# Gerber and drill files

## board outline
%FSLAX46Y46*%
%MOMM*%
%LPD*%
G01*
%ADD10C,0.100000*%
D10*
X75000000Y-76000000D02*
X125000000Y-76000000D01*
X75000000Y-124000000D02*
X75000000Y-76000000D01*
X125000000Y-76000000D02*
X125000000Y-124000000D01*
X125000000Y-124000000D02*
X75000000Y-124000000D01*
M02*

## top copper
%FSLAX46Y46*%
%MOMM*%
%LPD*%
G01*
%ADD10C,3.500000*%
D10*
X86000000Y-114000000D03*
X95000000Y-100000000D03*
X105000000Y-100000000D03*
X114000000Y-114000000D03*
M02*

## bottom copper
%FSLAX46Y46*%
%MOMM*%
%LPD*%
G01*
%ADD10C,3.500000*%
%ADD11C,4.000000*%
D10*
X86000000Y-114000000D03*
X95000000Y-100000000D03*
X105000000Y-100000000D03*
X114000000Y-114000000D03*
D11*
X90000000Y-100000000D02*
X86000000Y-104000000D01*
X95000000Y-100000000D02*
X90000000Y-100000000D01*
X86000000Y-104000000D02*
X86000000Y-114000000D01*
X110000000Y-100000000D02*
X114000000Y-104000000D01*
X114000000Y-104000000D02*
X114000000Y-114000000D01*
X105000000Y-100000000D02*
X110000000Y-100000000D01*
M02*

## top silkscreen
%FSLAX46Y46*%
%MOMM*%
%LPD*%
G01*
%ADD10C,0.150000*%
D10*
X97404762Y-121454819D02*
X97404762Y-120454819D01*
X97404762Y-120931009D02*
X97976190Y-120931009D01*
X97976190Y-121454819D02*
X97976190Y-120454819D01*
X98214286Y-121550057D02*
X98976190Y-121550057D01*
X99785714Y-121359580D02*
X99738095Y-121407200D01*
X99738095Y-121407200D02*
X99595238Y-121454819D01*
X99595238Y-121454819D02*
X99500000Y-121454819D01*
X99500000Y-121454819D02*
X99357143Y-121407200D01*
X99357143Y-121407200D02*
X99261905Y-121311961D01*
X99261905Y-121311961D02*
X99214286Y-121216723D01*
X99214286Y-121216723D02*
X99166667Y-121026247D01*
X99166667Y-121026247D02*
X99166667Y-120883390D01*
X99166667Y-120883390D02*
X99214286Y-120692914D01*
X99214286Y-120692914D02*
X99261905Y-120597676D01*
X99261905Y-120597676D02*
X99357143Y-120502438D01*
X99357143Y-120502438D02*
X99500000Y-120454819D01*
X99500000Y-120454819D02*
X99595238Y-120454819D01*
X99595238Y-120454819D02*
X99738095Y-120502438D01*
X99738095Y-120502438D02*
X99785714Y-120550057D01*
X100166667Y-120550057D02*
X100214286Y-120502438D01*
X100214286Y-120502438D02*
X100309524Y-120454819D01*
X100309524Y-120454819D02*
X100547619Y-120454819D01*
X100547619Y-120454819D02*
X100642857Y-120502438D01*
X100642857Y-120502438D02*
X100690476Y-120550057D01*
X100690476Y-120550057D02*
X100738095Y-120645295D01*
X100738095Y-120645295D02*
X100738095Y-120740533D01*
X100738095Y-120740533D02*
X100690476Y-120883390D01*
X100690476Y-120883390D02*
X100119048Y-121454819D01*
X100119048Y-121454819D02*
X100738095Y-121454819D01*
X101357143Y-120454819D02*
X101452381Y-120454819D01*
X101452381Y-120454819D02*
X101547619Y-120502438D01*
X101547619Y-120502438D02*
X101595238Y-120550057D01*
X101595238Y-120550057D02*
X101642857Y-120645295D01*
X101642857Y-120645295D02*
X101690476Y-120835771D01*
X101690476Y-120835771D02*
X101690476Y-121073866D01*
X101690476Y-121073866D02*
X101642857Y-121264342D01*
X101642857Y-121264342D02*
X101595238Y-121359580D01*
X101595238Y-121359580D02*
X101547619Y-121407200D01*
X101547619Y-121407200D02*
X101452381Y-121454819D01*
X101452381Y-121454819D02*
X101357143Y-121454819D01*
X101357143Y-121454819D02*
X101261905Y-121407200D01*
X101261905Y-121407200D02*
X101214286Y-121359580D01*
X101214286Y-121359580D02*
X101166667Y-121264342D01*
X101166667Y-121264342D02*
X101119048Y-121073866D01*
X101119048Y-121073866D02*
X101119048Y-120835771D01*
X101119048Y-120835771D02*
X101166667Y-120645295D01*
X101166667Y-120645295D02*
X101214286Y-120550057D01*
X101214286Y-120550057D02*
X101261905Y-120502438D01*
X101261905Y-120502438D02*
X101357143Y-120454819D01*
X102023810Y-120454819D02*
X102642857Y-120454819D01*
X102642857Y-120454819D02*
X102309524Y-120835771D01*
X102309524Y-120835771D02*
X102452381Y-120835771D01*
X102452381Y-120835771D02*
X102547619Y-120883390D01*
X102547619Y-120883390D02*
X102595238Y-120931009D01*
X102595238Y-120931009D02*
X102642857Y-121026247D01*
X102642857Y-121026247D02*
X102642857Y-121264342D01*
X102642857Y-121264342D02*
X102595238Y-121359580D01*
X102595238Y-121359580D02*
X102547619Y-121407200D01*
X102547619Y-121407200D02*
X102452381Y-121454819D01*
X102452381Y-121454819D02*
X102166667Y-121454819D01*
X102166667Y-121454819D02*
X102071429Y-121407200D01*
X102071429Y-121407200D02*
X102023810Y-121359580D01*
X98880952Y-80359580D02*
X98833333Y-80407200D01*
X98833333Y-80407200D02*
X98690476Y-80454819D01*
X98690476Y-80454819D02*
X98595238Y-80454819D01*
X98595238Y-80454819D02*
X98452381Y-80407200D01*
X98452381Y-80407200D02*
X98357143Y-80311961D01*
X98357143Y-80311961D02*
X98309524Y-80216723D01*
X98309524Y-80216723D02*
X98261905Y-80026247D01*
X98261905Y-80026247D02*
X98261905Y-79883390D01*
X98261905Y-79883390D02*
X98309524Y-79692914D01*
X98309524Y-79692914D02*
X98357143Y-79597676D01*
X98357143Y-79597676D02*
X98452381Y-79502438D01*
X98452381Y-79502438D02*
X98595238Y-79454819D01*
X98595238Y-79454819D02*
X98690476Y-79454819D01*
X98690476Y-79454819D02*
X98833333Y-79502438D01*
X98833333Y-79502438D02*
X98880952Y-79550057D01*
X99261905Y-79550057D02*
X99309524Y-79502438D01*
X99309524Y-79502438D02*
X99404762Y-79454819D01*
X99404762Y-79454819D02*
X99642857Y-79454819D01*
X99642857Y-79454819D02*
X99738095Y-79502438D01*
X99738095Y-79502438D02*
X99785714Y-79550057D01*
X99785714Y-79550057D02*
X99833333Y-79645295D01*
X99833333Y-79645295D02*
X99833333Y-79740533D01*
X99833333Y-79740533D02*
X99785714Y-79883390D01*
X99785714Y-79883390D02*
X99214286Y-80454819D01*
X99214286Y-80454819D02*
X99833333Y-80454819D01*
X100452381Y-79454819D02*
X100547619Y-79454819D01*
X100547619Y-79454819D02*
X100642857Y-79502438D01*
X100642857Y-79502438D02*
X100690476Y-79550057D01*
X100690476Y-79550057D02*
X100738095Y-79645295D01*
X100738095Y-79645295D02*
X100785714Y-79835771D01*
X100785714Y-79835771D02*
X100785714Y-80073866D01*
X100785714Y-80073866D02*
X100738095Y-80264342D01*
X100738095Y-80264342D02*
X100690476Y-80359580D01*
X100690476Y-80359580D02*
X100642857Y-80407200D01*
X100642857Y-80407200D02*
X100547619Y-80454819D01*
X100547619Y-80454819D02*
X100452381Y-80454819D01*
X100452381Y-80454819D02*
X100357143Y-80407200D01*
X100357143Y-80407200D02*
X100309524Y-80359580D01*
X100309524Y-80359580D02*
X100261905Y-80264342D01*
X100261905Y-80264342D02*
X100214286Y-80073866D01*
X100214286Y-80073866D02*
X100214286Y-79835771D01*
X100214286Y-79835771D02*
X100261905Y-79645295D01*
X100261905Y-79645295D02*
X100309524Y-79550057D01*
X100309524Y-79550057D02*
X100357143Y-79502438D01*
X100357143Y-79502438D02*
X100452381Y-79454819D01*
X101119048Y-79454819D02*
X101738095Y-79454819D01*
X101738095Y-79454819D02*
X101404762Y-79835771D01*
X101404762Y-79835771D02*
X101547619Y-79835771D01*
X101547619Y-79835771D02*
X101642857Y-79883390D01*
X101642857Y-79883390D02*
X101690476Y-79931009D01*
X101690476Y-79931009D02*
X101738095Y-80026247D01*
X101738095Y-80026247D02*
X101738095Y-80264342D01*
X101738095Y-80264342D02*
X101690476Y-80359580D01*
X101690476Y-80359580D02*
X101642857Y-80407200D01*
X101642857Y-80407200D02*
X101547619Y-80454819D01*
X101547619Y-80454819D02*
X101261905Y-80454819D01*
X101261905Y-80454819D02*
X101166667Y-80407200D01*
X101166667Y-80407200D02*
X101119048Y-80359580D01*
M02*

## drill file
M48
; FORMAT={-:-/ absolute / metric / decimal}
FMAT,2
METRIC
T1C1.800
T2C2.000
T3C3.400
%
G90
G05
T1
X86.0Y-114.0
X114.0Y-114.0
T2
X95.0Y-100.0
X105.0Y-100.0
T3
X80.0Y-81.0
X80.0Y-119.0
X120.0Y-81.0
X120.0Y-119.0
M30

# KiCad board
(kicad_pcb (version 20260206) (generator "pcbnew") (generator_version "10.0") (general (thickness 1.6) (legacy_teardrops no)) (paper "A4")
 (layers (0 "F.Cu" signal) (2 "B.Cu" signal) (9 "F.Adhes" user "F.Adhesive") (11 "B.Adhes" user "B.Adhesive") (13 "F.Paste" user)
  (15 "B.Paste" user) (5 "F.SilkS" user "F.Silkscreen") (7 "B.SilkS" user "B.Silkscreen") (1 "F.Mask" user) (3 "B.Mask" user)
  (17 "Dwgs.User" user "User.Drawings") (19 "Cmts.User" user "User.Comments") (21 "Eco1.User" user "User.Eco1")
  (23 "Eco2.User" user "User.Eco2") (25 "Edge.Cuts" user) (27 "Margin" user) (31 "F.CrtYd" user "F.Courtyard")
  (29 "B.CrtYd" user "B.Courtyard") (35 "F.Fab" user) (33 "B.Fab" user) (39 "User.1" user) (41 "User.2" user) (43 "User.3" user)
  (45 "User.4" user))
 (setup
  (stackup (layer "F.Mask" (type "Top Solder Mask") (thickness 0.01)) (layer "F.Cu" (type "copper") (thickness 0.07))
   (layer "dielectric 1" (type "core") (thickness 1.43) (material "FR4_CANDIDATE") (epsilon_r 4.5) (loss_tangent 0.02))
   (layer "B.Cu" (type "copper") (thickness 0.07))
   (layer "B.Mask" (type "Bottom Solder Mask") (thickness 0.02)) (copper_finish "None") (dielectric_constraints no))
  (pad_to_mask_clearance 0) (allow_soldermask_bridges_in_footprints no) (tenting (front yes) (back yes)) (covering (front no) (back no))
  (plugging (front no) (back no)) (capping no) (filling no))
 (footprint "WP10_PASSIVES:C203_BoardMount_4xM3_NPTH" (layer "F.Cu") (at 100 100)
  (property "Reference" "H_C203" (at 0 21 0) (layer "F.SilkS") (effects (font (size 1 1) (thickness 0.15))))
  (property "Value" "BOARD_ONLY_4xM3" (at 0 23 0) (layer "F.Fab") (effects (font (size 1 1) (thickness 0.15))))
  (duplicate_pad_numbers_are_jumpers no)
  (pad "" np_thru_hole circle (at -20 -19) (size 3.4 3.4) (drill 3.4) (layers "*.Cu" "*.Mask"))
  (pad "" np_thru_hole circle (at -20 19) (size 3.4 3.4) (drill 3.4) (layers "*.Cu" "*.Mask"))
  (pad "" np_thru_hole circle (at 20 -19) (size 3.4 3.4) (drill 3.4) (layers "*.Cu" "*.Mask"))
  (pad "" np_thru_hole circle (at 20 19) (size 3.4 3.4) (drill 3.4) (layers "*.Cu" "*.Mask")))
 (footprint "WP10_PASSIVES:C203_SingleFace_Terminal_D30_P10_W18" (layer "F.Cu") (at 100 100)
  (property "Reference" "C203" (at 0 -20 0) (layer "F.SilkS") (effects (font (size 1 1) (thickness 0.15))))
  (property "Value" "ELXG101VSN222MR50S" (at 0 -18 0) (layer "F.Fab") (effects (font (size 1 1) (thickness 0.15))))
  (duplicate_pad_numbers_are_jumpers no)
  (pad "1" thru_hole circle (at -14 14) (size 3.5 3.5) (drill 1.8) (layers "*.Cu" "*.Mask") (remove_unused_layers no)
   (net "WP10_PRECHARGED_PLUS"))
  (pad "1" thru_hole circle (at -5 0) (size 3.5 3.5) (drill 2) (layers "*.Mask" "B.Cu") (remove_unused_layers no)
   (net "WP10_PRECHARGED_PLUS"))
  (pad "2" thru_hole circle (at 5 0) (size 3.5 3.5) (drill 2) (layers "*.Mask" "B.Cu") (remove_unused_layers no) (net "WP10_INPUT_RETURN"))
  (pad "2" thru_hole circle (at 14 14) (size 3.5 3.5) (drill 1.8) (layers "*.Cu" "*.Mask") (remove_unused_layers no)
   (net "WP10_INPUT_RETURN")))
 (gr_line (start 75 76) (end 125 76) (stroke (width 0.1) (type default)) (layer "Edge.Cuts"))
 (gr_line (start 75 124) (end 75 76) (stroke (width 0.1) (type default)) (layer "Edge.Cuts"))
 (gr_line (start 125 76) (end 125 124) (stroke (width 0.1) (type default)) (layer "Edge.Cuts"))
 (gr_line (start 125 124) (end 75 124) (stroke (width 0.1) (type default)) (layer "Edge.Cuts"))
 (segment (start 90 100) (end 86 104) (width 4) (layer "B.Cu") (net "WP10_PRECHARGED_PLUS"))
 (segment (start 95 100) (end 90 100) (width 4) (layer "B.Cu") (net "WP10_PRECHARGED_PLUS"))
 (segment (start 86 104) (end 86 114) (width 4) (layer "B.Cu") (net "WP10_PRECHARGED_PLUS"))
 (segment (start 110 100) (end 114 104) (width 4) (layer "B.Cu") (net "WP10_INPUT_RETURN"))
 (segment (start 114 104) (end 114 114) (width 4) (layer "B.Cu") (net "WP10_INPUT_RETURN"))
 (segment (start 105 100) (end 110 100) (width 4) (layer "B.Cu") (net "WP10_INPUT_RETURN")))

